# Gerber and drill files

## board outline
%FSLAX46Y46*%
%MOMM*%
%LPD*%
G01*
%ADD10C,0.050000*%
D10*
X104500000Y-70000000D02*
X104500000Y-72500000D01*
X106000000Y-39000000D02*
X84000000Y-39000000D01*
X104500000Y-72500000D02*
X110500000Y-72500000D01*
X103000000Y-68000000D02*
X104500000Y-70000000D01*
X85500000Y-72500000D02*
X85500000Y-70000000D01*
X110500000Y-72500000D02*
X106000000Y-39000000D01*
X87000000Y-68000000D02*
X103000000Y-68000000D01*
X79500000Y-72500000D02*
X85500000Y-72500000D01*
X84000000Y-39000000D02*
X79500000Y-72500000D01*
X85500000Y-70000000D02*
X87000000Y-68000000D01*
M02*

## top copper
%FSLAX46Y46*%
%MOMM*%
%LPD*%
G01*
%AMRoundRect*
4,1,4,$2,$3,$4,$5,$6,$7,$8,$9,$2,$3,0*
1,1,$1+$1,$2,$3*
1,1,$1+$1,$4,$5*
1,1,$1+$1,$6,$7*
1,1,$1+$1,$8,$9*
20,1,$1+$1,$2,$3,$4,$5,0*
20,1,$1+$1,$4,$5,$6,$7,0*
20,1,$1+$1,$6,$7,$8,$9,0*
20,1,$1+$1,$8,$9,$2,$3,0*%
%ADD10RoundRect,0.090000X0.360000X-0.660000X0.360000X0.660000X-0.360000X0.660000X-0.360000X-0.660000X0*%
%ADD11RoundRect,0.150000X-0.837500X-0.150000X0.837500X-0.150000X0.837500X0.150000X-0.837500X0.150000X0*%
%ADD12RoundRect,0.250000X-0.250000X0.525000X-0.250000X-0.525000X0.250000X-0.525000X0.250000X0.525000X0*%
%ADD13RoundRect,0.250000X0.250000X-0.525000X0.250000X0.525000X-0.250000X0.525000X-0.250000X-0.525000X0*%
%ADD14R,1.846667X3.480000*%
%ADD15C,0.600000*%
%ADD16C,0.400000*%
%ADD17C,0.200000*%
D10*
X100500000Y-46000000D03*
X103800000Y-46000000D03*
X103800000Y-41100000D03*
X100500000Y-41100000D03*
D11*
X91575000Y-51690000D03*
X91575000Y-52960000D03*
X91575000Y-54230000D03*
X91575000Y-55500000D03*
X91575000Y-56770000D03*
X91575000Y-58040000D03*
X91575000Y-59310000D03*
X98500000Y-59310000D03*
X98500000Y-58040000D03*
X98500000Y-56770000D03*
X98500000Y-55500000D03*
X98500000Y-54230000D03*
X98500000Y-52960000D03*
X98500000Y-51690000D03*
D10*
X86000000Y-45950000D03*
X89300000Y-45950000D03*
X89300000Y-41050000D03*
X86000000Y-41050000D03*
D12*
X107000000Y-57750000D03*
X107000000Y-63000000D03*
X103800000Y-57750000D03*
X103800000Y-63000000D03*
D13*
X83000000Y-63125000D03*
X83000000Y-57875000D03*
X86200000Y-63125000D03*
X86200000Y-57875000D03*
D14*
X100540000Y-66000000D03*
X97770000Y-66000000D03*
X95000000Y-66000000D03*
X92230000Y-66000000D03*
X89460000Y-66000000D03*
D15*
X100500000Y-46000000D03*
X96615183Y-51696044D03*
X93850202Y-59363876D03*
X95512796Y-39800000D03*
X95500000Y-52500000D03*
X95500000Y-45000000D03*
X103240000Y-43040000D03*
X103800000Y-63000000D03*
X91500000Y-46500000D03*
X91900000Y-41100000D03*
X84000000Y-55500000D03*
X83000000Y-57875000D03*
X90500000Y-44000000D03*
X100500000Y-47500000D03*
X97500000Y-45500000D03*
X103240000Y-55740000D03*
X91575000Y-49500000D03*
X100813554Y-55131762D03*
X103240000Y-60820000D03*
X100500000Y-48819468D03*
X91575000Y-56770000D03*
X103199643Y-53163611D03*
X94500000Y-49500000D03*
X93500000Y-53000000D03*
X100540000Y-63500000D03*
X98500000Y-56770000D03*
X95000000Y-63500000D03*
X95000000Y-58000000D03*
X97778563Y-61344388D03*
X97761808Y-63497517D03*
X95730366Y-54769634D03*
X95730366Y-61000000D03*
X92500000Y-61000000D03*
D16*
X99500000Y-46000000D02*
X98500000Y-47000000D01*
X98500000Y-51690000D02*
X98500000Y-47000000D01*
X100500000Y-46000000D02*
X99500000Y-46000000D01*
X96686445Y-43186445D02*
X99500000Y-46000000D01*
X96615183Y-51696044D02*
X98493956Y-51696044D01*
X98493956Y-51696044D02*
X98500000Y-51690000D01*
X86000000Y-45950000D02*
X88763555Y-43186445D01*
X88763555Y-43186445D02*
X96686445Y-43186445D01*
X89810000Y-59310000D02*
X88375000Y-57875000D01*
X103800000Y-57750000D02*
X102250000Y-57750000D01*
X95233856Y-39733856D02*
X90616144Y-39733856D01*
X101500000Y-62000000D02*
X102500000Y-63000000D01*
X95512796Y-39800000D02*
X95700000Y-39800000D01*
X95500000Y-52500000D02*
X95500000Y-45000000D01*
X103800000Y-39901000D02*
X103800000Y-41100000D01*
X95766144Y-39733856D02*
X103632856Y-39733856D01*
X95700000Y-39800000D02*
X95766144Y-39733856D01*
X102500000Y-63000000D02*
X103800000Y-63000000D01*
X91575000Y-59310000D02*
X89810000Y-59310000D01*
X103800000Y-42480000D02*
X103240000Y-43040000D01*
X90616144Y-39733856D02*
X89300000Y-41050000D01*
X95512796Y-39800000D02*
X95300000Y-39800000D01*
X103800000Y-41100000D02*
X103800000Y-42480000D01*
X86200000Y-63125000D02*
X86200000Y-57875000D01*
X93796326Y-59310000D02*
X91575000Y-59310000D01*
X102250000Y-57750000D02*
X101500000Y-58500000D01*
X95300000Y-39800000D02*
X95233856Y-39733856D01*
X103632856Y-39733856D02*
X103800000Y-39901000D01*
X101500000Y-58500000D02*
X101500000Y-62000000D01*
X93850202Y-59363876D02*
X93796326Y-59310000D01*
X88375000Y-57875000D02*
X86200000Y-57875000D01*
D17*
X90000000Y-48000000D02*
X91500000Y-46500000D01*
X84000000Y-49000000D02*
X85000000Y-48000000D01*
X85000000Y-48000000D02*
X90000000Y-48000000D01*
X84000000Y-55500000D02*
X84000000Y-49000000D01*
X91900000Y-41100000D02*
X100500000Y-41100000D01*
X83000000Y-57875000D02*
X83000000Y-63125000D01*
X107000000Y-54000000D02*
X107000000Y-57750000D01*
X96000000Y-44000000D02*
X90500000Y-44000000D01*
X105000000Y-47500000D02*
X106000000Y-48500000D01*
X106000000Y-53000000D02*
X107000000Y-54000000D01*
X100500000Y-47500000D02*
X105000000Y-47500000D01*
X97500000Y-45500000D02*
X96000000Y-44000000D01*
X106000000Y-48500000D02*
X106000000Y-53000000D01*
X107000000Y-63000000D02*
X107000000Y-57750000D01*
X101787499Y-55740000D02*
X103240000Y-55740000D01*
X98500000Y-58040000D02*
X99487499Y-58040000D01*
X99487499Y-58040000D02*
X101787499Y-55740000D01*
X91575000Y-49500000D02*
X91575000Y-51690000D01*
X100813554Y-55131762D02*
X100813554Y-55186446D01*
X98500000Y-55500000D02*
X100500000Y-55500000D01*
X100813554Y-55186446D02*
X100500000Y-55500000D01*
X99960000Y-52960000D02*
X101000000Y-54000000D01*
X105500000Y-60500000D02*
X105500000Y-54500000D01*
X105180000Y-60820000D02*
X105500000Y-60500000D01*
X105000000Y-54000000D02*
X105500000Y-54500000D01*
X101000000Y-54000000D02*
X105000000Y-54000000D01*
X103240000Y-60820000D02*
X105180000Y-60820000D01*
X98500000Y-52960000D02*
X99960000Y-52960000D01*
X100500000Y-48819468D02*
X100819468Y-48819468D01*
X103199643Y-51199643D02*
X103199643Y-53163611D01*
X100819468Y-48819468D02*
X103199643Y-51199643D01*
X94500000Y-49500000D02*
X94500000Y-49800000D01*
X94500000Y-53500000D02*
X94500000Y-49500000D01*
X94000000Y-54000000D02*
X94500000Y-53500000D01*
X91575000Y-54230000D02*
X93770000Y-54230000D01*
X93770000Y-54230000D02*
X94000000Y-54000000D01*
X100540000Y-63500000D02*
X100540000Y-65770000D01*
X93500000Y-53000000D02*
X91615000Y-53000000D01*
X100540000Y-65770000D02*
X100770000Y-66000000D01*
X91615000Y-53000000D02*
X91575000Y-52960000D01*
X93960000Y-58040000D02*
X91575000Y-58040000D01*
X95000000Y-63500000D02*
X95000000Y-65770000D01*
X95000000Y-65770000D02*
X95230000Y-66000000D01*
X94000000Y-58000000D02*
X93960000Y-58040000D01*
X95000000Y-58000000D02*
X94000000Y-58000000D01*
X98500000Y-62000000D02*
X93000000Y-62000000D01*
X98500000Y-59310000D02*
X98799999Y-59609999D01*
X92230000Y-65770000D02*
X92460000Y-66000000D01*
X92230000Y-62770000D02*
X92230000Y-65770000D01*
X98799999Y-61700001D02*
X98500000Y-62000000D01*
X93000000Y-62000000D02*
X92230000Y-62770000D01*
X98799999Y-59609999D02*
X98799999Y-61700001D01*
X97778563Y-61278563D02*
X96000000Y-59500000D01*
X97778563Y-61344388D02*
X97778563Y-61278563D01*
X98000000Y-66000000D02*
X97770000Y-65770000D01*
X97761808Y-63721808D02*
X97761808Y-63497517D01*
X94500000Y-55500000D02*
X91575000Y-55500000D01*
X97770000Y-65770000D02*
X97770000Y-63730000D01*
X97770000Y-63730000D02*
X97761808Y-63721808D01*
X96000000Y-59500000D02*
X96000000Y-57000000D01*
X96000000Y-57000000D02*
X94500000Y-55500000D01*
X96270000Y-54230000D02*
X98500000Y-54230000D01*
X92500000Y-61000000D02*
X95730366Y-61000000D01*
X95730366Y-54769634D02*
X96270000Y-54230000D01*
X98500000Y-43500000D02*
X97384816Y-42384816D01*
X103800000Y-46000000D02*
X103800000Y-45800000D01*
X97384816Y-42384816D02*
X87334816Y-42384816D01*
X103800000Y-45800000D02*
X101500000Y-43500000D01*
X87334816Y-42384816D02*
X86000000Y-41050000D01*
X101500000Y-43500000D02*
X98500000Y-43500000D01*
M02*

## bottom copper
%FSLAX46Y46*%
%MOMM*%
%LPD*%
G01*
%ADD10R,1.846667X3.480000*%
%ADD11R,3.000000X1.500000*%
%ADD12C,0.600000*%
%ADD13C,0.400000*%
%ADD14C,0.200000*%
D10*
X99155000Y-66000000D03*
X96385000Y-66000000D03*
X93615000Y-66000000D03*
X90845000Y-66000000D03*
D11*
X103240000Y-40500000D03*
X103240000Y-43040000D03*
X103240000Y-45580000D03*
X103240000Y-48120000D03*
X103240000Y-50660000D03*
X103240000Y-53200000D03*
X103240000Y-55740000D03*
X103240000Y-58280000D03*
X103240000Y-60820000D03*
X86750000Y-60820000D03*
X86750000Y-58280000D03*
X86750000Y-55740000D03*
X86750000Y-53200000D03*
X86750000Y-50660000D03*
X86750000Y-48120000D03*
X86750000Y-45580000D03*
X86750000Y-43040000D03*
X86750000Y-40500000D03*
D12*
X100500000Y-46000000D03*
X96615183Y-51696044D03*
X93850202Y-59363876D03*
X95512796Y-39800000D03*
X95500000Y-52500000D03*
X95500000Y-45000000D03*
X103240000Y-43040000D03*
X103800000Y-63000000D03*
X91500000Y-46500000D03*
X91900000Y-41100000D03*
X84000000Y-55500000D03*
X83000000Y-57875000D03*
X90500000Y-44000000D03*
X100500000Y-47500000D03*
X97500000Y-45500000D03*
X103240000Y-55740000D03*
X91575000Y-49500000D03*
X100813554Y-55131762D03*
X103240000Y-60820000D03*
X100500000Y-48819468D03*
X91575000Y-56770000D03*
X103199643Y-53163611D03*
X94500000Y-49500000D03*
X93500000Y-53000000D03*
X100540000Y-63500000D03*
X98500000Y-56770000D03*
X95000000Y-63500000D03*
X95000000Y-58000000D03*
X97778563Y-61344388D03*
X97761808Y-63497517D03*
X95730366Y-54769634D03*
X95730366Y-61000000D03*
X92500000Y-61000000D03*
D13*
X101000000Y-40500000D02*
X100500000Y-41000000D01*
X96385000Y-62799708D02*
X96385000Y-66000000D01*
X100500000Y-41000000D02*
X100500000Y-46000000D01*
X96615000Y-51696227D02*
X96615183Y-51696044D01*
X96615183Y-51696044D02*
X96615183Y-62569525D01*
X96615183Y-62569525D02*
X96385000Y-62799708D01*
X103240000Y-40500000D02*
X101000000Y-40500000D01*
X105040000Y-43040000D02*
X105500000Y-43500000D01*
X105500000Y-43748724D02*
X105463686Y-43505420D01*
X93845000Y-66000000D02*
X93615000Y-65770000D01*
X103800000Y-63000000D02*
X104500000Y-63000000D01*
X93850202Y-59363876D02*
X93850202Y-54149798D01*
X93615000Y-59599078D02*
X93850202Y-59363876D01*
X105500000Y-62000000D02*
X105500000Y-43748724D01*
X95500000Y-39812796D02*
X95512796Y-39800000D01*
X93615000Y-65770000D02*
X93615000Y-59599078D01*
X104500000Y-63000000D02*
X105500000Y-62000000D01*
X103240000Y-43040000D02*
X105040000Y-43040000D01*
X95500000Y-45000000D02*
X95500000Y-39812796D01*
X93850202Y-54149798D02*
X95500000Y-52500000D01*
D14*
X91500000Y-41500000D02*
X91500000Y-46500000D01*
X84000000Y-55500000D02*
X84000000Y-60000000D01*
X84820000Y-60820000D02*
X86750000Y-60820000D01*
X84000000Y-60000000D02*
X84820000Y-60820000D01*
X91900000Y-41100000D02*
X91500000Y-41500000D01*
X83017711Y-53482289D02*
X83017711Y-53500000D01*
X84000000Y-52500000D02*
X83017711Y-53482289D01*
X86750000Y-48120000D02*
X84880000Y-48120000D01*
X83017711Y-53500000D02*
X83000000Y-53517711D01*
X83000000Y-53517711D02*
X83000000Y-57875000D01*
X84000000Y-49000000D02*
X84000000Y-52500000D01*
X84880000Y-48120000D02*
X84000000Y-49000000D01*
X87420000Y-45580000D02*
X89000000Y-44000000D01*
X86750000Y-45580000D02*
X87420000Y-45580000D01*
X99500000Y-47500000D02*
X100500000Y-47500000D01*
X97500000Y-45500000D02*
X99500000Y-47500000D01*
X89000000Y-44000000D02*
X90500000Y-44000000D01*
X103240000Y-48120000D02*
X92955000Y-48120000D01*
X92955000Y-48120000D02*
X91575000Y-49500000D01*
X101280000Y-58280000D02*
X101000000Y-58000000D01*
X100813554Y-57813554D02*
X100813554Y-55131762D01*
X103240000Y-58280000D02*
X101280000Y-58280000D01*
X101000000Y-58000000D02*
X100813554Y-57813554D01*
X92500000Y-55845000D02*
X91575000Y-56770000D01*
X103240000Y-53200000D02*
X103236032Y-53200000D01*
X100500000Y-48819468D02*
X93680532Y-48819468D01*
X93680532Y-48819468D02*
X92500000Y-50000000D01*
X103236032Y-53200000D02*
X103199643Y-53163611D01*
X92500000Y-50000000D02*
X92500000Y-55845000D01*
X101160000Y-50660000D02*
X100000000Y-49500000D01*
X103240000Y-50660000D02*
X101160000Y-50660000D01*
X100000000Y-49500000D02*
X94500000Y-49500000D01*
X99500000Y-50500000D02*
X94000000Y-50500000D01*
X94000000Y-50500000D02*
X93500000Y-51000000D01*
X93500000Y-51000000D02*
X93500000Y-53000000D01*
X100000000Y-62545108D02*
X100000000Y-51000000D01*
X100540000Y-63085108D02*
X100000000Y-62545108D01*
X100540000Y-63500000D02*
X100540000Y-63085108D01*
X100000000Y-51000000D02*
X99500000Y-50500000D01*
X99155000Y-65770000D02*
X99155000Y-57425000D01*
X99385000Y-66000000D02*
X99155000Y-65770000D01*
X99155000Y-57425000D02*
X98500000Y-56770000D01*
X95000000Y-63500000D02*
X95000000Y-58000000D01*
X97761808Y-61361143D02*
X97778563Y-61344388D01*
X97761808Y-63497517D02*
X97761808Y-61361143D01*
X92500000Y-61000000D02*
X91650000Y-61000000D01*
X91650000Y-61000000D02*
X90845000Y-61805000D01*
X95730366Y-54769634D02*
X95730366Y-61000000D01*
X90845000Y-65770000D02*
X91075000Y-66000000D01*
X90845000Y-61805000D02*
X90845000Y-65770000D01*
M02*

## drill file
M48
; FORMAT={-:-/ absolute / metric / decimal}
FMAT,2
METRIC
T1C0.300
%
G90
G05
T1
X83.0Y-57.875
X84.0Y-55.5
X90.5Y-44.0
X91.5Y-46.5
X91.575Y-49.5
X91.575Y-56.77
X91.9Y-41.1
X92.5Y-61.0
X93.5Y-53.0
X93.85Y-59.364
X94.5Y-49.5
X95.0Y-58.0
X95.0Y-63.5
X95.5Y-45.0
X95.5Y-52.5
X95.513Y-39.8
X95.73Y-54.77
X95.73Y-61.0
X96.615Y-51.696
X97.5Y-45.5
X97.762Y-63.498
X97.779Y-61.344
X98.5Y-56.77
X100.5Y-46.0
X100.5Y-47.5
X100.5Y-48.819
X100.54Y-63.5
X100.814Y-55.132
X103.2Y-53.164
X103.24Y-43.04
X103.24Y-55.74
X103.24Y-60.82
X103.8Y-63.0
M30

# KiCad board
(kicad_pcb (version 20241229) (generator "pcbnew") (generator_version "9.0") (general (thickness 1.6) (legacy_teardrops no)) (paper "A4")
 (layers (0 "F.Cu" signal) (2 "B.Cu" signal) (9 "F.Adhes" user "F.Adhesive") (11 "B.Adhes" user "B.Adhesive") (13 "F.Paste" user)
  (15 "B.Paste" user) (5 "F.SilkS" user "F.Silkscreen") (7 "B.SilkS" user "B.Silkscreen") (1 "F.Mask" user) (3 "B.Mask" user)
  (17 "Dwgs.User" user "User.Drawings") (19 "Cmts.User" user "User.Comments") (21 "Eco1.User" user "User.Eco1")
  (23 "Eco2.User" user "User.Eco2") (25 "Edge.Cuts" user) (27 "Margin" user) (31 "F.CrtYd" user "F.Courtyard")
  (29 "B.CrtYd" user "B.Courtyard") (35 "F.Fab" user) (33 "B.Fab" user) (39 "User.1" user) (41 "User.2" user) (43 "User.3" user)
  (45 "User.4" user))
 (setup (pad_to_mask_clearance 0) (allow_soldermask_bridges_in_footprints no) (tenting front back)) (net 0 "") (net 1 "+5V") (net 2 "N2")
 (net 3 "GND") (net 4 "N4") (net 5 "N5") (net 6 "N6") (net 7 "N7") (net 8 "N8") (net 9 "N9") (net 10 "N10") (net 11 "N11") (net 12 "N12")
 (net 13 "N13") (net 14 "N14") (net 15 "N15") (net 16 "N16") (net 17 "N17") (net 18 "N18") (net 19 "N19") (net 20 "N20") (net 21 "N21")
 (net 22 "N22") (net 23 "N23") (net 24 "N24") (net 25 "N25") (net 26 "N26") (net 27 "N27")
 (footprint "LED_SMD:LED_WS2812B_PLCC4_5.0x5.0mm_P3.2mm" (layer "F.Cu") (at 102.15 43.55 90)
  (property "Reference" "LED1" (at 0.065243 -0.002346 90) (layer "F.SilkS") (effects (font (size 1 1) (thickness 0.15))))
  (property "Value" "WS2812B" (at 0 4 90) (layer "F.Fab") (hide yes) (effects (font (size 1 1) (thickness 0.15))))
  (pad "1" smd roundrect (at -2.45 -1.65 90) (size 1.5 0.9) (layers "F.Cu" "F.Mask" "F.Paste") (roundrect_rratio 0.1) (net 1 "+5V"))
  (pad "2" smd roundrect (at -2.45 1.65 90) (size 1.5 0.9) (layers "F.Cu" "F.Mask" "F.Paste") (roundrect_rratio 0.1) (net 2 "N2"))
  (pad "3" smd roundrect (at 2.45 1.65 90) (size 1.5 0.9) (layers "F.Cu" "F.Mask" "F.Paste") (roundrect_rratio 0.1) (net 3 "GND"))
  (pad "4" smd roundrect (at 2.45 -1.65 90) (size 1.5 0.9) (layers "F.Cu" "F.Mask" "F.Paste") (roundrect_rratio 0.1) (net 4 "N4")))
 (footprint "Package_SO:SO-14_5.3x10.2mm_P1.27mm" (layer "F.Cu") (at 95.0375 55.5)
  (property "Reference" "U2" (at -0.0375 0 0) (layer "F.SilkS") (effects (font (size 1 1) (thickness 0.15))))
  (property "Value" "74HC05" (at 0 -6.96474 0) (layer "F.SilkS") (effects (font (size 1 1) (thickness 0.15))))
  (pad "1" smd roundrect (at -3.4625 -3.81) (size 1.975 0.6) (layers "F.Cu" "F.Mask" "F.Paste") (roundrect_rratio 0.25) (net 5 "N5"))
  (pad "2" smd roundrect (at -3.4625 -2.54) (size 1.975 0.6) (layers "F.Cu" "F.Mask" "F.Paste") (roundrect_rratio 0.25) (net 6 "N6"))
  (pad "3" smd roundrect (at -3.4625 -1.27) (size 1.975 0.6) (layers "F.Cu" "F.Mask" "F.Paste") (roundrect_rratio 0.25) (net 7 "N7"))
  (pad "4" smd roundrect (at -3.4625 0) (size 1.975 0.6) (layers "F.Cu" "F.Mask" "F.Paste") (roundrect_rratio 0.25) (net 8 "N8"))
  (pad "5" smd roundrect (at -3.4625 1.27) (size 1.975 0.6) (layers "F.Cu" "F.Mask" "F.Paste") (roundrect_rratio 0.25) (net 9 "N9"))
  (pad "6" smd roundrect (at -3.4625 2.54) (size 1.975 0.6) (layers "F.Cu" "F.Mask" "F.Paste") (roundrect_rratio 0.25) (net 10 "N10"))
  (pad "7" smd roundrect (at -3.4625 3.81) (size 1.975 0.6) (layers "F.Cu" "F.Mask" "F.Paste") (roundrect_rratio 0.25) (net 3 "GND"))
  (pad "8" smd roundrect (at 3.4625 3.81) (size 1.975 0.6) (layers "F.Cu" "F.Mask" "F.Paste") (roundrect_rratio 0.25) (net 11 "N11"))
  (pad "9" smd roundrect (at 3.4625 2.54) (size 1.975 0.6) (layers "F.Cu" "F.Mask" "F.Paste") (roundrect_rratio 0.25) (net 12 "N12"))
  (pad "10" smd roundrect (at 3.4625 1.27) (size 1.975 0.6) (layers "F.Cu" "F.Mask" "F.Paste") (roundrect_rratio 0.25) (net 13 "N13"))
  (pad "11" smd roundrect (at 3.4625 0) (size 1.975 0.6) (layers "F.Cu" "F.Mask" "F.Paste") (roundrect_rratio 0.25) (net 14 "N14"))
  (pad "12" smd roundrect (at 3.4625 -1.27) (size 1.975 0.6) (layers "F.Cu" "F.Mask" "F.Paste") (roundrect_rratio 0.25) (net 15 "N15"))
  (pad "13" smd roundrect (at 3.4625 -2.54) (size 1.975 0.6) (layers "F.Cu" "F.Mask" "F.Paste") (roundrect_rratio 0.25) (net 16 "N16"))
  (pad "14" smd roundrect (at 3.4625 -3.81) (size 1.975 0.6) (layers "F.Cu" "F.Mask" "F.Paste") (roundrect_rratio 0.25) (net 1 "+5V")))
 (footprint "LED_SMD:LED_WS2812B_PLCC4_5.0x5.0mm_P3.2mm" (layer "F.Cu") (at 87.65 43.5 90)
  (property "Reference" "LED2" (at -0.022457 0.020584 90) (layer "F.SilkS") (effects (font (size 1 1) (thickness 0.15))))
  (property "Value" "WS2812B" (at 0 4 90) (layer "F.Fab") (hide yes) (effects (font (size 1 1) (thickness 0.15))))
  (pad "1" smd roundrect (at -2.45 -1.65 90) (size 1.5 0.9) (layers "F.Cu" "F.Mask" "F.Paste") (roundrect_rratio 0.1) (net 1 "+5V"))
  (pad "2" smd roundrect (at -2.45 1.65 90) (size 1.5 0.9) (layers "F.Cu" "F.Mask" "F.Paste") (roundrect_rratio 0.1) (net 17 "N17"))
  (pad "3" smd roundrect (at 2.45 1.65 90) (size 1.5 0.9) (layers "F.Cu" "F.Mask" "F.Paste") (roundrect_rratio 0.1) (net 3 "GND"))
  (pad "4" smd roundrect (at 2.45 -1.65 90) (size 1.5 0.9) (layers "F.Cu" "F.Mask" "F.Paste") (roundrect_rratio 0.1) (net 2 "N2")))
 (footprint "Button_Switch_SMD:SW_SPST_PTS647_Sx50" (layer "F.Cu") (at 105.4 60.375 -90)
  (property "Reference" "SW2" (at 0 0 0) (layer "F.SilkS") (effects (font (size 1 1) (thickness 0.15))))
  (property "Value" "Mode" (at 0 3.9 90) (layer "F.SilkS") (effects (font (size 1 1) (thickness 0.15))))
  (pad "1" smd roundrect (at -2.625 -1.6 270) (size 1.55 1) (layers "F.Cu" "F.Mask" "F.Paste") (roundrect_rratio 0.25) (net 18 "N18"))
  (pad "1" smd roundrect (at 2.625 -1.6 270) (size 1.55 1) (layers "F.Cu" "F.Mask" "F.Paste") (roundrect_rratio 0.25) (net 18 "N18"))
  (pad "2" smd roundrect (at -2.625 1.6 270) (size 1.55 1) (layers "F.Cu" "F.Mask" "F.Paste") (roundrect_rratio 0.25) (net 3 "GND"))
  (pad "2" smd roundrect (at 2.625 1.6 270) (size 1.55 1) (layers "F.Cu" "F.Mask" "F.Paste") (roundrect_rratio 0.25) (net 3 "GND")))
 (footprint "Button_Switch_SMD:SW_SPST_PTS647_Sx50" (layer "F.Cu") (at 84.6 60.5 90)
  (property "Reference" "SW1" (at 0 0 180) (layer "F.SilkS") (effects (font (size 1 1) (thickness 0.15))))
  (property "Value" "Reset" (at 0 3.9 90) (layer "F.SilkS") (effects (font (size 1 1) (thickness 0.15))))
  (pad "1" smd roundrect (at -2.625 -1.6 90) (size 1.55 1) (layers "F.Cu" "F.Mask" "F.Paste") (roundrect_rratio 0.25) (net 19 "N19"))
  (pad "1" smd roundrect (at 2.625 -1.6 90) (size 1.55 1) (layers "F.Cu" "F.Mask" "F.Paste") (roundrect_rratio 0.25) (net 19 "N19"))
  (pad "2" smd roundrect (at -2.625 1.6 90) (size 1.55 1) (layers "F.Cu" "F.Mask" "F.Paste") (roundrect_rratio 0.25) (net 3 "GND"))
  (pad "2" smd roundrect (at 2.625 1.6 90) (size 1.55 1) (layers "F.Cu" "F.Mask" "F.Paste") (roundrect_rratio 0.25) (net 3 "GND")))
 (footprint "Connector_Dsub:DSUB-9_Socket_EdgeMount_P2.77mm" (layer "F.Cu") (at 95 66)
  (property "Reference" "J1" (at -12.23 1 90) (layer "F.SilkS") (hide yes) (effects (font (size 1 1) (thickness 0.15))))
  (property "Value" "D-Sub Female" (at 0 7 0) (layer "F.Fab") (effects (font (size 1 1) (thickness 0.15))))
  (pad "1" smd rect (at 5.54 0) (size 1.846667 3.48) (layers "F.Cu" "F.Mask" "F.Paste") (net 6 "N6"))
  (pad "2" smd rect (at 2.77 0) (size 1.846667 3.48) (layers "F.Cu" "F.Mask" "F.Paste") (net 8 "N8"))
  (pad "3" smd rect (at 0 0) (size 1.846667 3.48) (layers "F.Cu" "F.Mask" "F.Paste") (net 10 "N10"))
  (pad "4" smd rect (at -2.77 0) (size 1.846667 3.48) (layers "F.Cu" "F.Mask" "F.Paste") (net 11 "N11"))
  (pad "5" smd rect (at -5.54 0) (size 1.846667 3.48) (layers "F.Cu" "F.Mask" "F.Paste") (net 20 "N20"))
  (pad "6" smd rect (at 4.155 0) (size 1.846667 3.48) (layers "B.Cu" "B.Mask" "B.Paste") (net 13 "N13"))
  (pad "7" smd rect (at 1.385 0) (size 1.846667 3.48) (layers "B.Cu" "B.Mask" "B.Paste") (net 1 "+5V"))
  (pad "8" smd rect (at -1.385 0) (size 1.846667 3.48) (layers "B.Cu" "B.Mask" "B.Paste") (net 3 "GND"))
  (pad "9" smd rect (at -4.155 0) (size 1.846667 3.48) (layers "B.Cu" "B.Mask" "B.Paste") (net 15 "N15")))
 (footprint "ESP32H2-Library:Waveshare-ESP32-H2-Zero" (layer "B.Cu") (at 95.5 50.41 180)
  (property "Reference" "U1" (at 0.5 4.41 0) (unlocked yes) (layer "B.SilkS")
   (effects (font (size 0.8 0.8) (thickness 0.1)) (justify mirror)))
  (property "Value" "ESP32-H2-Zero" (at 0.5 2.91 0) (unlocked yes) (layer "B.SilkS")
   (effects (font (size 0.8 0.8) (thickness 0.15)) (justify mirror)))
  (pad "1" smd rect (at -7.74 9.91 180) (size 3 1.5) (layers "B.Cu" "B.Mask" "B.Paste") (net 1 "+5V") (thermal_bridge_angle 45))
  (pad "2" smd rect (at -7.74 7.37 180) (size 3 1.5) (layers "B.Cu" "B.Mask" "B.Paste") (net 3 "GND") (thermal_bridge_angle 45))
  (pad "3" smd rect (at -7.74 4.83 180) (size 3 1.5) (layers "B.Cu" "B.Mask" "B.Paste") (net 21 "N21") (thermal_bridge_angle 45))
  (pad "4" smd rect (at -7.74 2.29 180) (size 3 1.5) (layers "B.Cu" "B.Mask" "B.Paste") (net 5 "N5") (thermal_bridge_angle 45))
  (pad "5" smd rect (at -7.74 -0.25 180) (size 3 1.5) (layers "B.Cu" "B.Mask" "B.Paste") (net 7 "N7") (thermal_bridge_angle 45))
  (pad "6" smd rect (at -7.74 -2.79 180) (size 3 1.5) (layers "B.Cu" "B.Mask" "B.Paste") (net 9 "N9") (thermal_bridge_angle 45))
  (pad "7" smd rect (at -7.74 -5.33 180) (size 3 1.5) (layers "B.Cu" "B.Mask" "B.Paste") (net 12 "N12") (thermal_bridge_angle 45))
  (pad "8" smd rect (at -7.74 -7.87 180) (size 3 1.5) (layers "B.Cu" "B.Mask" "B.Paste") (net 14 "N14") (thermal_bridge_angle 45))
  (pad "9" smd rect (at -7.74 -10.41 180) (size 3 1.5) (layers "B.Cu" "B.Mask" "B.Paste") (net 16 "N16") (thermal_bridge_angle 45))
  (pad "10" smd rect (at 8.75 -10.41 180) (size 3 1.5) (layers "B.Cu" "B.Mask" "B.Paste") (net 4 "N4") (thermal_bridge_angle 45))
  (pad "11" smd rect (at 8.75 -7.87 180) (size 3 1.5) (layers "B.Cu" "B.Mask" "B.Paste") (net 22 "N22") (thermal_bridge_angle 45))
  (pad "12" smd rect (at 8.75 -5.33 180) (size 3 1.5) (layers "B.Cu" "B.Mask" "B.Paste") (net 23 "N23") (thermal_bridge_angle 45))
  (pad "13" smd rect (at 8.75 -2.79 180) (size 3 1.5) (layers "B.Cu" "B.Mask" "B.Paste") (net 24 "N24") (thermal_bridge_angle 45))
  (pad "14" smd rect (at 8.75 -0.25 180) (size 3 1.5) (layers "B.Cu" "B.Mask" "B.Paste") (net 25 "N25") (thermal_bridge_angle 45))
  (pad "15" smd rect (at 8.75 2.29 180) (size 3 1.5) (layers "B.Cu" "B.Mask" "B.Paste") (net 19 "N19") (thermal_bridge_angle 45))
  (pad "16" smd rect (at 8.75 4.83 180) (size 3 1.5) (layers "B.Cu" "B.Mask" "B.Paste") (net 18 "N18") (thermal_bridge_angle 45))
  (pad "17" smd rect (at 8.75 7.37 180) (size 3 1.5) (layers "B.Cu" "B.Mask" "B.Paste") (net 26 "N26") (thermal_bridge_angle 45))
  (pad "18" smd rect (at 8.75 9.91 180) (size 3 1.5) (layers "B.Cu" "B.Mask" "B.Paste") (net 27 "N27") (thermal_bridge_angle 45)))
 (gr_line (start 104.5 70) (end 104.5 72.5) (stroke (width 0.05) (type default)) (layer "Edge.Cuts"))
 (gr_line (start 106 39) (end 84 39) (stroke (width 0.05) (type default)) (layer "Edge.Cuts"))
 (gr_line (start 104.5 72.5) (end 110.5 72.5) (stroke (width 0.05) (type default)) (layer "Edge.Cuts"))
 (gr_line (start 103 68) (end 104.5 70) (stroke (width 0.05) (type default)) (layer "Edge.Cuts"))
 (gr_line (start 85.5 72.5) (end 85.5 70) (stroke (width 0.05) (type default)) (layer "Edge.Cuts"))
 (gr_line (start 110.5 72.5) (end 106 39) (stroke (width 0.05) (type default)) (layer "Edge.Cuts"))
 (gr_line (start 87 68) (end 103 68) (stroke (width 0.05) (type default)) (layer "Edge.Cuts"))
 (gr_line (start 79.5 72.5) (end 85.5 72.5) (stroke (width 0.05) (type default)) (layer "Edge.Cuts"))
 (gr_line (start 84 39) (end 79.5 72.5) (stroke (width 0.05) (type default)) (layer "Edge.Cuts"))
 (gr_line (start 85.5 70) (end 87 68) (stroke (width 0.05) (type default)) (layer "Edge.Cuts"))
 (segment (start 99.5 46) (end 98.5 47) (width 0.4) (layer "F.Cu") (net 1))
 (segment (start 98.5 51.69) (end 98.5 47) (width 0.4) (layer "F.Cu") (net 1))
 (segment (start 100.5 46) (end 99.5 46) (width 0.4) (layer "F.Cu") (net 1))
 (segment (start 96.686445 43.186445) (end 99.5 46) (width 0.4) (layer "F.Cu") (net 1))
 (segment (start 96.615183 51.696044) (end 98.493956 51.696044) (width 0.4) (layer "F.Cu") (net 1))
 (segment (start 98.493956 51.696044) (end 98.5 51.69) (width 0.4) (layer "F.Cu") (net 1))
 (segment (start 86 45.95) (end 88.763555 43.186445) (width 0.4) (layer "F.Cu") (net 1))
 (segment (start 88.763555 43.186445) (end 96.686445 43.186445) (width 0.4) (layer "F.Cu") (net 1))
 (via (at 100.5 46) (size 0.6) (drill 0.3) (layers "F.Cu" "B.Cu") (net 1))
 (via (at 96.615183 51.696044) (size 0.6) (drill 0.3) (layers "F.Cu" "B.Cu") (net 1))
 (segment (start 101 40.5) (end 100.5 41) (width 0.4) (layer "B.Cu") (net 1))
 (segment (start 96.385 62.799708) (end 96.385 66) (width 0.4) (layer "B.Cu") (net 1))
 (segment (start 100.5 41) (end 100.5 46) (width 0.4) (layer "B.Cu") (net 1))
 (segment (start 96.615 51.696227) (end 96.615183 51.696044) (width 0.4) (layer "B.Cu") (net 1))
 (segment (start 96.615183 51.696044) (end 96.615183 62.569525) (width 0.4) (layer "B.Cu") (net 1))
 (segment (start 96.615183 62.569525) (end 96.385 62.799708) (width 0.4) (layer "B.Cu") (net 1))
 (segment (start 103.24 40.5) (end 101 40.5) (width 0.4) (layer "B.Cu") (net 1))
 (segment (start 89.81 59.31) (end 88.375 57.875) (width 0.4) (layer "F.Cu") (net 3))
 (segment (start 103.8 57.75) (end 102.25 57.75) (width 0.4) (layer "F.Cu") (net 3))
 (segment (start 95.233856 39.733856) (end 90.616144 39.733856) (width 0.4) (layer "F.Cu") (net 3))
 (segment (start 101.5 62) (end 102.5 63) (width 0.4) (layer "F.Cu") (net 3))
 (segment (start 95.512796 39.8) (end 95.7 39.8) (width 0.4) (layer "F.Cu") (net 3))
 (segment (start 95.5 52.5) (end 95.5 45) (width 0.4) (layer "F.Cu") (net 3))
 (segment (start 103.8 39.901) (end 103.8 41.1) (width 0.4) (layer "F.Cu") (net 3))
 (segment (start 95.766144 39.733856) (end 103.632856 39.733856) (width 0.4) (layer "F.Cu") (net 3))
 (segment (start 95.7 39.8) (end 95.766144 39.733856) (width 0.4) (layer "F.Cu") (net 3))
 (segment (start 102.5 63) (end 103.8 63) (width 0.4) (layer "F.Cu") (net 3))
 (segment (start 91.575 59.31) (end 89.81 59.31) (width 0.4) (layer "F.Cu") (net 3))
 (segment (start 103.8 42.48) (end 103.24 43.04) (width 0.4) (layer "F.Cu") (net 3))
 (segment (start 90.616144 39.733856) (end 89.3 41.05) (width 0.4) (layer "F.Cu") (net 3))
 (segment (start 95.512796 39.8) (end 95.3 39.8) (width 0.4) (layer "F.Cu") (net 3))
 (segment (start 103.8 41.1) (end 103.8 42.48) (width 0.4) (layer "F.Cu") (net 3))
 (segment (start 86.2 63.125) (end 86.2 57.875) (width 0.4) (layer "F.Cu") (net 3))
 (segment (start 93.796326 59.31) (end 91.575 59.31) (width 0.4) (layer "F.Cu") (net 3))
 (segment (start 102.25 57.75) (end 101.5 58.5) (width 0.4) (layer "F.Cu") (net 3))
 (segment (start 95.3 39.8) (end 95.233856 39.733856) (width 0.4) (layer "F.Cu") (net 3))
 (segment (start 103.632856 39.733856) (end 103.8 39.901) (width 0.4) (layer "F.Cu") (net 3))
 (segment (start 101.5 58.5) (end 101.5 62) (width 0.4) (layer "F.Cu") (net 3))
 (segment (start 93.850202 59.363876) (end 93.796326 59.31) (width 0.4) (layer "F.Cu") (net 3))
 (segment (start 88.375 57.875) (end 86.2 57.875) (width 0.4) (layer "F.Cu") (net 3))
 (via (at 93.850202 59.363876) (size 0.6) (drill 0.3) (layers "F.Cu" "B.Cu") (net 3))
 (via (at 95.512796 39.8) (size 0.6) (drill 0.3) (layers "F.Cu" "B.Cu") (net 3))
 (via (at 95.5 52.5) (size 0.6) (drill 0.3) (layers "F.Cu" "B.Cu") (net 3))
 (via (at 95.5 45) (size 0.6) (drill 0.3) (layers "F.Cu" "B.Cu") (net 3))
 (via (at 103.24 43.04) (size 0.6) (drill 0.3) (layers "F.Cu" "B.Cu") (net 3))
 (via (at 103.8 63) (size 0.6) (drill 0.3) (layers "F.Cu" "B.Cu") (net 3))
 (segment (start 105.04 43.04) (end 105.5 43.5) (width 0.4) (layer "B.Cu") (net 3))
 (segment (start 105.5 43.748724) (end 105.463686 43.50542) (width 0.4) (layer "B.Cu") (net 3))
 (segment (start 93.845 66) (end 93.615 65.77) (width 0.4) (layer "B.Cu") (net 3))
 (segment (start 103.8 63) (end 104.5 63) (width 0.4) (layer "B.Cu") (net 3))
 (segment (start 93.850202 59.363876) (end 93.850202 54.149798) (width 0.4) (layer "B.Cu") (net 3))
 (segment (start 93.615 59.599078) (end 93.850202 59.363876) (width 0.4) (layer "B.Cu") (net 3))
 (segment (start 105.5 62) (end 105.5 43.748724) (width 0.4) (layer "B.Cu") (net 3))
 (segment (start 95.5 39.812796) (end 95.512796 39.8) (width 0.4) (layer "B.Cu") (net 3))
 (segment (start 93.615 65.77) (end 93.615 59.599078) (width 0.4) (layer "B.Cu") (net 3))
 (segment (start 104.5 63) (end 105.5 62) (width 0.4) (layer "B.Cu") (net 3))
 (segment (start 103.24 43.04) (end 105.04 43.04) (width 0.4) (layer "B.Cu") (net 3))
 (segment (start 95.5 45) (end 95.5 39.812796) (width 0.4) (layer "B.Cu") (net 3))
 (segment (start 93.850202 54.149798) (end 95.5 52.5) (width 0.4) (layer "B.Cu") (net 3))
 (segment (start 90 48) (end 91.5 46.5) (width 0.2) (layer "F.Cu") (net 4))
 (segment (start 84 49) (end 85 48) (width 0.2) (layer "F.Cu") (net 4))
 (segment (start 85 48) (end 90 48) (width 0.2) (layer "F.Cu") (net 4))
 (segment (start 84 55.5) (end 84 49) (width 0.2) (layer "F.Cu") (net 4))
 (segment (start 91.9 41.1) (end 100.5 41.1) (width 0.2) (layer "F.Cu") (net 4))
 (via (at 91.5 46.5) (size 0.6) (drill 0.3) (layers "F.Cu" "B.Cu") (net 4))
 (via (at 91.9 41.1) (size 0.6) (drill 0.3) (layers "F.Cu" "B.Cu") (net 4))
 (via (at 84 55.5) (size 0.6) (drill 0.3) (layers "F.Cu" "B.Cu") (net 4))
 (segment (start 91.5 41.5) (end 91.5 46.5) (width 0.2) (layer "B.Cu") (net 4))
 (segment (start 84 55.5) (end 84 60) (width 0.2) (layer "B.Cu") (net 4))
 (segment (start 84.82 60.82) (end 86.75 60.82) (width 0.2) (layer "B.Cu") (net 4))
 (segment (start 84 60) (end 84.82 60.82) (width 0.2) (layer "B.Cu") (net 4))
 (segment (start 91.9 41.1) (end 91.5 41.5) (width 0.2) (layer "B.Cu") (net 4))
 (segment (start 83 57.875) (end 83 63.125) (width 0.2) (layer "F.Cu") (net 19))
 (via (at 83 57.875) (size 0.6) (drill 0.3) (layers "F.Cu" "B.Cu") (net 19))
 (segment (start 83.017711 53.482289) (end 83.017711 53.5) (width 0.2) (layer "B.Cu") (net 19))
 (segment (start 84 52.5) (end 83.017711 53.482289) (width 0.2) (layer "B.Cu") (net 19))
 (segment (start 86.75 48.12) (end 84.88 48.12) (width 0.2) (layer "B.Cu") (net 19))
 (segment (start 83.017711 53.5) (end 83 53.517711) (width 0.2) (layer "B.Cu") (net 19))
 (segment (start 83 53.517711) (end 83 57.875) (width 0.2) (layer "B.Cu") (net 19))
 (segment (start 84 49) (end 84 52.5) (width 0.2) (layer "B.Cu") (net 19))
 (segment (start 84.88 48.12) (end 84 49) (width 0.2) (layer "B.Cu") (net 19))
 (segment (start 107 54) (end 107 57.75) (width 0.2) (layer "F.Cu") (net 18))
 (segment (start 96 44) (end 90.5 44) (width 0.2) (layer "F.Cu") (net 18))
 (segment (start 105 47.5) (end 106 48.5) (width 0.2) (layer "F.Cu") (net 18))
 (segment (start 106 53) (end 107 54) (width 0.2) (layer "F.Cu") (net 18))
 (segment (start 100.5 47.5) (end 105 47.5) (width 0.2) (layer "F.Cu") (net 18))
 (segment (start 97.5 45.5) (end 96 44) (width 0.2) (layer "F.Cu") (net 18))
 (segment (start 106 48.5) (end 106 53) (width 0.2) (layer "F.Cu") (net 18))
 (segment (start 107 63) (end 107 57.75) (width 0.2) (layer "F.Cu") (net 18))
 (via (at 90.5 44) (size 0.6) (drill 0.3) (layers "F.Cu" "B.Cu") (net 18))
 (via (at 100.5 47.5) (size 0.6) (drill 0.3) (layers "F.Cu" "B.Cu") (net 18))
 (via (at 97.5 45.5) (size 0.6) (drill 0.3) (layers "F.Cu" "B.Cu") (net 18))
 (segment (start 87.42 45.58) (end 89 44) (width 0.2) (layer "B.Cu") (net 18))
 (segment (start 86.75 45.58) (end 87.42 45.58) (width 0.2) (layer "B.Cu") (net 18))
 (segment (start 99.5 47.5) (end 100.5 47.5) (width 0.2) (layer "B.Cu") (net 18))
 (segment (start 97.5 45.5) (end 99.5 47.5) (width 0.2) (layer "B.Cu") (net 18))
 (segment (start 89 44) (end 90.5 44) (width 0.2) (layer "B.Cu") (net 18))
 (segment (start 101.787499 55.74) (end 103.24 55.74) (width 0.2) (layer "F.Cu") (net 12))
 (segment (start 98.5 58.04) (end 99.487499 58.04) (width 0.2) (layer "F.Cu") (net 12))
 (segment (start 99.487499 58.04) (end 101.787499 55.74) (width 0.2) (layer "F.Cu") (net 12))
 (via (at 103.24 55.74) (size 0.6) (drill 0.3) (layers "F.Cu" "B.Cu") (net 12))
 (segment (start 91.575 49.5) (end 91.575 51.69) (width 0.2) (layer "F.Cu") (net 5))
 (via (at 91.575 49.5) (size 0.6) (drill 0.3) (layers "F.Cu" "B.Cu") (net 5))
 (segment (start 103.24 48.12) (end 92.955 48.12) (width 0.2) (layer "B.Cu") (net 5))
 (segment (start 92.955 48.12) (end 91.575 49.5) (width 0.2) (layer "B.Cu") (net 5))
 (segment (start 100.813554 55.131762) (end 100.813554 55.186446) (width 0.2) (layer "F.Cu") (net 14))
 (segment (start 98.5 55.5) (end 100.5 55.5) (width 0.2) (layer "F.Cu") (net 14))
 (segment (start 100.813554 55.186446) (end 100.5 55.5) (width 0.2) (layer "F.Cu") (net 14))
 (via (at 100.813554 55.131762) (size 0.6) (drill 0.3) (layers "F.Cu" "B.Cu") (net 14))
 (segment (start 101.28 58.28) (end 101 58) (width 0.2) (layer "B.Cu") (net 14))
 (segment (start 100.813554 57.813554) (end 100.813554 55.131762) (width 0.2) (layer "B.Cu") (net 14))
 (segment (start 103.24 58.28) (end 101.28 58.28) (width 0.2) (layer "B.Cu") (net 14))
 (segment (start 101 58) (end 100.813554 57.813554) (width 0.2) (layer "B.Cu") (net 14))
 (segment (start 99.96 52.96) (end 101 54) (width 0.2) (layer "F.Cu") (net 16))
 (segment (start 105.5 60.5) (end 105.5 54.5) (width 0.2) (layer "F.Cu") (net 16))
 (segment (start 105.18 60.82) (end 105.5 60.5) (width 0.2) (layer "F.Cu") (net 16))
 (segment (start 105 54) (end 105.5 54.5) (width 0.2) (layer "F.Cu") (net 16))
 (segment (start 101 54) (end 105 54) (width 0.2) (layer "F.Cu") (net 16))
 (segment (start 103.24 60.82) (end 105.18 60.82) (width 0.2) (layer "F.Cu") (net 16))
 (segment (start 98.5 52.96) (end 99.96 52.96) (width 0.2) (layer "F.Cu") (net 16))
 (via (at 103.24 60.82) (size 0.6) (drill 0.3) (layers "F.Cu" "B.Cu") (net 16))
 (segment (start 100.5 48.819468) (end 100.819468 48.819468) (width 0.2) (layer "F.Cu") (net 9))
 (segment (start 103.199643 51.199643) (end 103.199643 53.163611) (width 0.2) (layer "F.Cu") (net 9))
 (segment (start 100.819468 48.819468) (end 103.199643 51.199643) (width 0.2) (layer "F.Cu") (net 9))
 (via (at 100.5 48.819468) (size 0.6) (drill 0.3) (layers "F.Cu" "B.Cu") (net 9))
 (via (at 91.575 56.77) (size 0.6) (drill 0.3) (layers "F.Cu" "B.Cu") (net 9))
 (via (at 103.199643 53.163611) (size 0.6) (drill 0.3) (layers "F.Cu" "B.Cu") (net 9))
 (segment (start 92.5 55.845) (end 91.575 56.77) (width 0.2) (layer "B.Cu") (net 9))
 (segment (start 103.24 53.2) (end 103.236032 53.2) (width 0.2) (layer "B.Cu") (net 9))
 (segment (start 100.5 48.819468) (end 93.680532 48.819468) (width 0.2) (layer "B.Cu") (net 9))
 (segment (start 93.680532 48.819468) (end 92.5 50) (width 0.2) (layer "B.Cu") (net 9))
 (segment (start 103.236032 53.2) (end 103.199643 53.163611) (width 0.2) (layer "B.Cu") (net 9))
 (segment (start 92.5 50) (end 92.5 55.845) (width 0.2) (layer "B.Cu") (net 9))
 (segment (start 94.5 49.5) (end 94.5 49.8) (width 0.2) (layer "F.Cu") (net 7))
 (segment (start 94.5 53.5) (end 94.5 49.5) (width 0.2) (layer "F.Cu") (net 7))
 (segment (start 94 54) (end 94.5 53.5) (width 0.2) (layer "F.Cu") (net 7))
 (segment (start 91.575 54.23) (end 93.77 54.23) (width 0.2) (layer "F.Cu") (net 7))
 (segment (start 93.77 54.23) (end 94 54) (width 0.2) (layer "F.Cu") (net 7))
 (via (at 94.5 49.5) (size 0.6) (drill 0.3) (layers "F.Cu" "B.Cu") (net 7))
 (segment (start 101.16 50.66) (end 100 49.5) (width 0.2) (layer "B.Cu") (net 7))
 (segment (start 103.24 50.66) (end 101.16 50.66) (width 0.2) (layer "B.Cu") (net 7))
 (segment (start 100 49.5) (end 94.5 49.5) (width 0.2) (layer "B.Cu") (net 7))
 (segment (start 100.54 63.5) (end 100.54 65.77) (width 0.2) (layer "F.Cu") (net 6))
 (segment (start 93.5 53) (end 91.615 53) (width 0.2) (layer "F.Cu") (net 6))
 (segment (start 100.54 65.77) (end 100.77 66) (width 0.2) (layer "F.Cu") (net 6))
 (segment (start 91.615 53) (end 91.575 52.96) (width 0.2) (layer "F.Cu") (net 6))
 (via (at 93.5 53) (size 0.6) (drill 0.3) (layers "F.Cu" "B.Cu") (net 6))
 (via (at 100.54 63.5) (size 0.6) (drill 0.3) (layers "F.Cu" "B.Cu") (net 6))
 (segment (start 99.5 50.5) (end 94 50.5) (width 0.2) (layer "B.Cu") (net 6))
 (segment (start 94 50.5) (end 93.5 51) (width 0.2) (layer "B.Cu") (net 6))
 (segment (start 93.5 51) (end 93.5 53) (width 0.2) (layer "B.Cu") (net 6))
 (segment (start 100 62.545108) (end 100 51) (width 0.2) (layer "B.Cu") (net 6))
 (segment (start 100.54 63.085108) (end 100 62.545108) (width 0.2) (layer "B.Cu") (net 6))
 (segment (start 100.54 63.5) (end 100.54 63.085108) (width 0.2) (layer "B.Cu") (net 6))
 (segment (start 100 51) (end 99.5 50.5) (width 0.2) (layer "B.Cu") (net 6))
 (via (at 98.5 56.77) (size 0.6) (drill 0.3) (layers "F.Cu" "B.Cu") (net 13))
 (segment (start 99.155 65.77) (end 99.155 57.425) (width 0.2) (layer "B.Cu") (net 13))
 (segment (start 99.385 66) (end 99.155 65.77) (width 0.2) (layer "B.Cu") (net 13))
 (segment (start 99.155 57.425) (end 98.5 56.77) (width 0.2) (layer "B.Cu") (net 13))
 (segment (start 93.96 58.04) (end 91.575 58.04) (width 0.2) (layer "F.Cu") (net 10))
 (segment (start 95 63.5) (end 95 65.77) (width 0.2) (layer "F.Cu") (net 10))
 (segment (start 95 65.77) (end 95.23 66) (width 0.2) (layer "F.Cu") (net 10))
 (segment (start 94 58) (end 93.96 58.04) (width 0.2) (layer "F.Cu") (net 10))
 (segment (start 95 58) (end 94 58) (width 0.2) (layer "F.Cu") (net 10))
 (via (at 95 63.5) (size 0.6) (drill 0.3) (layers "F.Cu" "B.Cu") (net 10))
 (via (at 95 58) (size 0.6) (drill 0.3) (layers "F.Cu" "B.Cu") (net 10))
 (segment (start 95 63.5) (end 95 58) (width 0.2) (layer "B.Cu") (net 10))
 (segment (start 98.5 62) (end 93 62) (width 0.2) (layer "F.Cu") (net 11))
 (segment (start 98.5 59.31) (end 98.799999 59.609999) (width 0.2) (layer "F.Cu") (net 11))
 (segment (start 92.23 65.77) (end 92.46 66) (width 0.2) (layer "F.Cu") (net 11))
 (segment (start 92.23 62.77) (end 92.23 65.77) (width 0.2) (layer "F.Cu") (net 11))
 (segment (start 98.799999 61.700001) (end 98.5 62) (width 0.2) (layer "F.Cu") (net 11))
 (segment (start 93 62) (end 92.23 62.77) (width 0.2) (layer "F.Cu") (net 11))
 (segment (start 98.799999 59.609999) (end 98.799999 61.700001) (width 0.2) (layer "F.Cu") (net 11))
 (segment (start 97.778563 61.278563) (end 96 59.5) (width 0.2) (layer "F.Cu") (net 8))
 (segment (start 97.778563 61.344388) (end 97.778563 61.278563) (width 0.2) (layer "F.Cu") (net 8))
 (segment (start 98 66) (end 97.77 65.77) (width 0.2) (layer "F.Cu") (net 8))
 (segment (start 97.761808 63.721808) (end 97.761808 63.497517) (width 0.2) (layer "F.Cu") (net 8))
 (segment (start 94.5 55.5) (end 91.575 55.5) (width 0.2) (layer "F.Cu") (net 8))
 (segment (start 97.77 65.77) (end 97.77 63.73) (width 0.2) (layer "F.Cu") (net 8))
 (segment (start 97.77 63.73) (end 97.761808 63.721808) (width 0.2) (layer "F.Cu") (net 8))
 (segment (start 96 59.5) (end 96 57) (width 0.2) (layer "F.Cu") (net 8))
 (segment (start 96 57) (end 94.5 55.5) (width 0.2) (layer "F.Cu") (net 8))
 (via (at 97.778563 61.344388) (size 0.6) (drill 0.3) (layers "F.Cu" "B.Cu") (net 8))
 (via (at 97.761808 63.497517) (size 0.6) (drill 0.3) (layers "F.Cu" "B.Cu") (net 8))
 (segment (start 97.761808 61.361143) (end 97.778563 61.344388) (width 0.2) (layer "B.Cu") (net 8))
 (segment (start 97.761808 63.497517) (end 97.761808 61.361143) (width 0.2) (layer "B.Cu") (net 8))
 (segment (start 96.27 54.23) (end 98.5 54.23) (width 0.2) (layer "F.Cu") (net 15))
 (segment (start 92.5 61) (end 95.730366 61) (width 0.2) (layer "F.Cu") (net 15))
 (segment (start 95.730366 54.769634) (end 96.27 54.23) (width 0.2) (layer "F.Cu") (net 15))
 (via (at 95.730366 54.769634) (size 0.6) (drill 0.3) (layers "F.Cu" "B.Cu") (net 15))
 (via (at 95.730366 61) (size 0.6) (drill 0.3) (layers "F.Cu" "B.Cu") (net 15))
 (via (at 92.5 61) (size 0.6) (drill 0.3) (layers "F.Cu" "B.Cu") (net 15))
 (segment (start 92.5 61) (end 91.65 61) (width 0.2) (layer "B.Cu") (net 15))
 (segment (start 91.65 61) (end 90.845 61.805) (width 0.2) (layer "B.Cu") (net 15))
 (segment (start 95.730366 54.769634) (end 95.730366 61) (width 0.2) (layer "B.Cu") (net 15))
 (segment (start 90.845 65.77) (end 91.075 66) (width 0.2) (layer "B.Cu") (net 15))
 (segment (start 90.845 61.805) (end 90.845 65.77) (width 0.2) (layer "B.Cu") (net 15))
 (segment (start 98.5 43.5) (end 97.384816 42.384816) (width 0.2) (layer "F.Cu") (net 2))
 (segment (start 103.8 46) (end 103.8 45.8) (width 0.2) (layer "F.Cu") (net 2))
 (segment (start 97.384816 42.384816) (end 87.334816 42.384816) (width 0.2) (layer "F.Cu") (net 2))
 (segment (start 103.8 45.8) (end 101.5 43.5) (width 0.2) (layer "F.Cu") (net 2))
 (segment (start 87.334816 42.384816) (end 86 41.05) (width 0.2) (layer "F.Cu") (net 2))
 (segment (start 101.5 43.5) (end 98.5 43.5) (width 0.2) (layer "F.Cu") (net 2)))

